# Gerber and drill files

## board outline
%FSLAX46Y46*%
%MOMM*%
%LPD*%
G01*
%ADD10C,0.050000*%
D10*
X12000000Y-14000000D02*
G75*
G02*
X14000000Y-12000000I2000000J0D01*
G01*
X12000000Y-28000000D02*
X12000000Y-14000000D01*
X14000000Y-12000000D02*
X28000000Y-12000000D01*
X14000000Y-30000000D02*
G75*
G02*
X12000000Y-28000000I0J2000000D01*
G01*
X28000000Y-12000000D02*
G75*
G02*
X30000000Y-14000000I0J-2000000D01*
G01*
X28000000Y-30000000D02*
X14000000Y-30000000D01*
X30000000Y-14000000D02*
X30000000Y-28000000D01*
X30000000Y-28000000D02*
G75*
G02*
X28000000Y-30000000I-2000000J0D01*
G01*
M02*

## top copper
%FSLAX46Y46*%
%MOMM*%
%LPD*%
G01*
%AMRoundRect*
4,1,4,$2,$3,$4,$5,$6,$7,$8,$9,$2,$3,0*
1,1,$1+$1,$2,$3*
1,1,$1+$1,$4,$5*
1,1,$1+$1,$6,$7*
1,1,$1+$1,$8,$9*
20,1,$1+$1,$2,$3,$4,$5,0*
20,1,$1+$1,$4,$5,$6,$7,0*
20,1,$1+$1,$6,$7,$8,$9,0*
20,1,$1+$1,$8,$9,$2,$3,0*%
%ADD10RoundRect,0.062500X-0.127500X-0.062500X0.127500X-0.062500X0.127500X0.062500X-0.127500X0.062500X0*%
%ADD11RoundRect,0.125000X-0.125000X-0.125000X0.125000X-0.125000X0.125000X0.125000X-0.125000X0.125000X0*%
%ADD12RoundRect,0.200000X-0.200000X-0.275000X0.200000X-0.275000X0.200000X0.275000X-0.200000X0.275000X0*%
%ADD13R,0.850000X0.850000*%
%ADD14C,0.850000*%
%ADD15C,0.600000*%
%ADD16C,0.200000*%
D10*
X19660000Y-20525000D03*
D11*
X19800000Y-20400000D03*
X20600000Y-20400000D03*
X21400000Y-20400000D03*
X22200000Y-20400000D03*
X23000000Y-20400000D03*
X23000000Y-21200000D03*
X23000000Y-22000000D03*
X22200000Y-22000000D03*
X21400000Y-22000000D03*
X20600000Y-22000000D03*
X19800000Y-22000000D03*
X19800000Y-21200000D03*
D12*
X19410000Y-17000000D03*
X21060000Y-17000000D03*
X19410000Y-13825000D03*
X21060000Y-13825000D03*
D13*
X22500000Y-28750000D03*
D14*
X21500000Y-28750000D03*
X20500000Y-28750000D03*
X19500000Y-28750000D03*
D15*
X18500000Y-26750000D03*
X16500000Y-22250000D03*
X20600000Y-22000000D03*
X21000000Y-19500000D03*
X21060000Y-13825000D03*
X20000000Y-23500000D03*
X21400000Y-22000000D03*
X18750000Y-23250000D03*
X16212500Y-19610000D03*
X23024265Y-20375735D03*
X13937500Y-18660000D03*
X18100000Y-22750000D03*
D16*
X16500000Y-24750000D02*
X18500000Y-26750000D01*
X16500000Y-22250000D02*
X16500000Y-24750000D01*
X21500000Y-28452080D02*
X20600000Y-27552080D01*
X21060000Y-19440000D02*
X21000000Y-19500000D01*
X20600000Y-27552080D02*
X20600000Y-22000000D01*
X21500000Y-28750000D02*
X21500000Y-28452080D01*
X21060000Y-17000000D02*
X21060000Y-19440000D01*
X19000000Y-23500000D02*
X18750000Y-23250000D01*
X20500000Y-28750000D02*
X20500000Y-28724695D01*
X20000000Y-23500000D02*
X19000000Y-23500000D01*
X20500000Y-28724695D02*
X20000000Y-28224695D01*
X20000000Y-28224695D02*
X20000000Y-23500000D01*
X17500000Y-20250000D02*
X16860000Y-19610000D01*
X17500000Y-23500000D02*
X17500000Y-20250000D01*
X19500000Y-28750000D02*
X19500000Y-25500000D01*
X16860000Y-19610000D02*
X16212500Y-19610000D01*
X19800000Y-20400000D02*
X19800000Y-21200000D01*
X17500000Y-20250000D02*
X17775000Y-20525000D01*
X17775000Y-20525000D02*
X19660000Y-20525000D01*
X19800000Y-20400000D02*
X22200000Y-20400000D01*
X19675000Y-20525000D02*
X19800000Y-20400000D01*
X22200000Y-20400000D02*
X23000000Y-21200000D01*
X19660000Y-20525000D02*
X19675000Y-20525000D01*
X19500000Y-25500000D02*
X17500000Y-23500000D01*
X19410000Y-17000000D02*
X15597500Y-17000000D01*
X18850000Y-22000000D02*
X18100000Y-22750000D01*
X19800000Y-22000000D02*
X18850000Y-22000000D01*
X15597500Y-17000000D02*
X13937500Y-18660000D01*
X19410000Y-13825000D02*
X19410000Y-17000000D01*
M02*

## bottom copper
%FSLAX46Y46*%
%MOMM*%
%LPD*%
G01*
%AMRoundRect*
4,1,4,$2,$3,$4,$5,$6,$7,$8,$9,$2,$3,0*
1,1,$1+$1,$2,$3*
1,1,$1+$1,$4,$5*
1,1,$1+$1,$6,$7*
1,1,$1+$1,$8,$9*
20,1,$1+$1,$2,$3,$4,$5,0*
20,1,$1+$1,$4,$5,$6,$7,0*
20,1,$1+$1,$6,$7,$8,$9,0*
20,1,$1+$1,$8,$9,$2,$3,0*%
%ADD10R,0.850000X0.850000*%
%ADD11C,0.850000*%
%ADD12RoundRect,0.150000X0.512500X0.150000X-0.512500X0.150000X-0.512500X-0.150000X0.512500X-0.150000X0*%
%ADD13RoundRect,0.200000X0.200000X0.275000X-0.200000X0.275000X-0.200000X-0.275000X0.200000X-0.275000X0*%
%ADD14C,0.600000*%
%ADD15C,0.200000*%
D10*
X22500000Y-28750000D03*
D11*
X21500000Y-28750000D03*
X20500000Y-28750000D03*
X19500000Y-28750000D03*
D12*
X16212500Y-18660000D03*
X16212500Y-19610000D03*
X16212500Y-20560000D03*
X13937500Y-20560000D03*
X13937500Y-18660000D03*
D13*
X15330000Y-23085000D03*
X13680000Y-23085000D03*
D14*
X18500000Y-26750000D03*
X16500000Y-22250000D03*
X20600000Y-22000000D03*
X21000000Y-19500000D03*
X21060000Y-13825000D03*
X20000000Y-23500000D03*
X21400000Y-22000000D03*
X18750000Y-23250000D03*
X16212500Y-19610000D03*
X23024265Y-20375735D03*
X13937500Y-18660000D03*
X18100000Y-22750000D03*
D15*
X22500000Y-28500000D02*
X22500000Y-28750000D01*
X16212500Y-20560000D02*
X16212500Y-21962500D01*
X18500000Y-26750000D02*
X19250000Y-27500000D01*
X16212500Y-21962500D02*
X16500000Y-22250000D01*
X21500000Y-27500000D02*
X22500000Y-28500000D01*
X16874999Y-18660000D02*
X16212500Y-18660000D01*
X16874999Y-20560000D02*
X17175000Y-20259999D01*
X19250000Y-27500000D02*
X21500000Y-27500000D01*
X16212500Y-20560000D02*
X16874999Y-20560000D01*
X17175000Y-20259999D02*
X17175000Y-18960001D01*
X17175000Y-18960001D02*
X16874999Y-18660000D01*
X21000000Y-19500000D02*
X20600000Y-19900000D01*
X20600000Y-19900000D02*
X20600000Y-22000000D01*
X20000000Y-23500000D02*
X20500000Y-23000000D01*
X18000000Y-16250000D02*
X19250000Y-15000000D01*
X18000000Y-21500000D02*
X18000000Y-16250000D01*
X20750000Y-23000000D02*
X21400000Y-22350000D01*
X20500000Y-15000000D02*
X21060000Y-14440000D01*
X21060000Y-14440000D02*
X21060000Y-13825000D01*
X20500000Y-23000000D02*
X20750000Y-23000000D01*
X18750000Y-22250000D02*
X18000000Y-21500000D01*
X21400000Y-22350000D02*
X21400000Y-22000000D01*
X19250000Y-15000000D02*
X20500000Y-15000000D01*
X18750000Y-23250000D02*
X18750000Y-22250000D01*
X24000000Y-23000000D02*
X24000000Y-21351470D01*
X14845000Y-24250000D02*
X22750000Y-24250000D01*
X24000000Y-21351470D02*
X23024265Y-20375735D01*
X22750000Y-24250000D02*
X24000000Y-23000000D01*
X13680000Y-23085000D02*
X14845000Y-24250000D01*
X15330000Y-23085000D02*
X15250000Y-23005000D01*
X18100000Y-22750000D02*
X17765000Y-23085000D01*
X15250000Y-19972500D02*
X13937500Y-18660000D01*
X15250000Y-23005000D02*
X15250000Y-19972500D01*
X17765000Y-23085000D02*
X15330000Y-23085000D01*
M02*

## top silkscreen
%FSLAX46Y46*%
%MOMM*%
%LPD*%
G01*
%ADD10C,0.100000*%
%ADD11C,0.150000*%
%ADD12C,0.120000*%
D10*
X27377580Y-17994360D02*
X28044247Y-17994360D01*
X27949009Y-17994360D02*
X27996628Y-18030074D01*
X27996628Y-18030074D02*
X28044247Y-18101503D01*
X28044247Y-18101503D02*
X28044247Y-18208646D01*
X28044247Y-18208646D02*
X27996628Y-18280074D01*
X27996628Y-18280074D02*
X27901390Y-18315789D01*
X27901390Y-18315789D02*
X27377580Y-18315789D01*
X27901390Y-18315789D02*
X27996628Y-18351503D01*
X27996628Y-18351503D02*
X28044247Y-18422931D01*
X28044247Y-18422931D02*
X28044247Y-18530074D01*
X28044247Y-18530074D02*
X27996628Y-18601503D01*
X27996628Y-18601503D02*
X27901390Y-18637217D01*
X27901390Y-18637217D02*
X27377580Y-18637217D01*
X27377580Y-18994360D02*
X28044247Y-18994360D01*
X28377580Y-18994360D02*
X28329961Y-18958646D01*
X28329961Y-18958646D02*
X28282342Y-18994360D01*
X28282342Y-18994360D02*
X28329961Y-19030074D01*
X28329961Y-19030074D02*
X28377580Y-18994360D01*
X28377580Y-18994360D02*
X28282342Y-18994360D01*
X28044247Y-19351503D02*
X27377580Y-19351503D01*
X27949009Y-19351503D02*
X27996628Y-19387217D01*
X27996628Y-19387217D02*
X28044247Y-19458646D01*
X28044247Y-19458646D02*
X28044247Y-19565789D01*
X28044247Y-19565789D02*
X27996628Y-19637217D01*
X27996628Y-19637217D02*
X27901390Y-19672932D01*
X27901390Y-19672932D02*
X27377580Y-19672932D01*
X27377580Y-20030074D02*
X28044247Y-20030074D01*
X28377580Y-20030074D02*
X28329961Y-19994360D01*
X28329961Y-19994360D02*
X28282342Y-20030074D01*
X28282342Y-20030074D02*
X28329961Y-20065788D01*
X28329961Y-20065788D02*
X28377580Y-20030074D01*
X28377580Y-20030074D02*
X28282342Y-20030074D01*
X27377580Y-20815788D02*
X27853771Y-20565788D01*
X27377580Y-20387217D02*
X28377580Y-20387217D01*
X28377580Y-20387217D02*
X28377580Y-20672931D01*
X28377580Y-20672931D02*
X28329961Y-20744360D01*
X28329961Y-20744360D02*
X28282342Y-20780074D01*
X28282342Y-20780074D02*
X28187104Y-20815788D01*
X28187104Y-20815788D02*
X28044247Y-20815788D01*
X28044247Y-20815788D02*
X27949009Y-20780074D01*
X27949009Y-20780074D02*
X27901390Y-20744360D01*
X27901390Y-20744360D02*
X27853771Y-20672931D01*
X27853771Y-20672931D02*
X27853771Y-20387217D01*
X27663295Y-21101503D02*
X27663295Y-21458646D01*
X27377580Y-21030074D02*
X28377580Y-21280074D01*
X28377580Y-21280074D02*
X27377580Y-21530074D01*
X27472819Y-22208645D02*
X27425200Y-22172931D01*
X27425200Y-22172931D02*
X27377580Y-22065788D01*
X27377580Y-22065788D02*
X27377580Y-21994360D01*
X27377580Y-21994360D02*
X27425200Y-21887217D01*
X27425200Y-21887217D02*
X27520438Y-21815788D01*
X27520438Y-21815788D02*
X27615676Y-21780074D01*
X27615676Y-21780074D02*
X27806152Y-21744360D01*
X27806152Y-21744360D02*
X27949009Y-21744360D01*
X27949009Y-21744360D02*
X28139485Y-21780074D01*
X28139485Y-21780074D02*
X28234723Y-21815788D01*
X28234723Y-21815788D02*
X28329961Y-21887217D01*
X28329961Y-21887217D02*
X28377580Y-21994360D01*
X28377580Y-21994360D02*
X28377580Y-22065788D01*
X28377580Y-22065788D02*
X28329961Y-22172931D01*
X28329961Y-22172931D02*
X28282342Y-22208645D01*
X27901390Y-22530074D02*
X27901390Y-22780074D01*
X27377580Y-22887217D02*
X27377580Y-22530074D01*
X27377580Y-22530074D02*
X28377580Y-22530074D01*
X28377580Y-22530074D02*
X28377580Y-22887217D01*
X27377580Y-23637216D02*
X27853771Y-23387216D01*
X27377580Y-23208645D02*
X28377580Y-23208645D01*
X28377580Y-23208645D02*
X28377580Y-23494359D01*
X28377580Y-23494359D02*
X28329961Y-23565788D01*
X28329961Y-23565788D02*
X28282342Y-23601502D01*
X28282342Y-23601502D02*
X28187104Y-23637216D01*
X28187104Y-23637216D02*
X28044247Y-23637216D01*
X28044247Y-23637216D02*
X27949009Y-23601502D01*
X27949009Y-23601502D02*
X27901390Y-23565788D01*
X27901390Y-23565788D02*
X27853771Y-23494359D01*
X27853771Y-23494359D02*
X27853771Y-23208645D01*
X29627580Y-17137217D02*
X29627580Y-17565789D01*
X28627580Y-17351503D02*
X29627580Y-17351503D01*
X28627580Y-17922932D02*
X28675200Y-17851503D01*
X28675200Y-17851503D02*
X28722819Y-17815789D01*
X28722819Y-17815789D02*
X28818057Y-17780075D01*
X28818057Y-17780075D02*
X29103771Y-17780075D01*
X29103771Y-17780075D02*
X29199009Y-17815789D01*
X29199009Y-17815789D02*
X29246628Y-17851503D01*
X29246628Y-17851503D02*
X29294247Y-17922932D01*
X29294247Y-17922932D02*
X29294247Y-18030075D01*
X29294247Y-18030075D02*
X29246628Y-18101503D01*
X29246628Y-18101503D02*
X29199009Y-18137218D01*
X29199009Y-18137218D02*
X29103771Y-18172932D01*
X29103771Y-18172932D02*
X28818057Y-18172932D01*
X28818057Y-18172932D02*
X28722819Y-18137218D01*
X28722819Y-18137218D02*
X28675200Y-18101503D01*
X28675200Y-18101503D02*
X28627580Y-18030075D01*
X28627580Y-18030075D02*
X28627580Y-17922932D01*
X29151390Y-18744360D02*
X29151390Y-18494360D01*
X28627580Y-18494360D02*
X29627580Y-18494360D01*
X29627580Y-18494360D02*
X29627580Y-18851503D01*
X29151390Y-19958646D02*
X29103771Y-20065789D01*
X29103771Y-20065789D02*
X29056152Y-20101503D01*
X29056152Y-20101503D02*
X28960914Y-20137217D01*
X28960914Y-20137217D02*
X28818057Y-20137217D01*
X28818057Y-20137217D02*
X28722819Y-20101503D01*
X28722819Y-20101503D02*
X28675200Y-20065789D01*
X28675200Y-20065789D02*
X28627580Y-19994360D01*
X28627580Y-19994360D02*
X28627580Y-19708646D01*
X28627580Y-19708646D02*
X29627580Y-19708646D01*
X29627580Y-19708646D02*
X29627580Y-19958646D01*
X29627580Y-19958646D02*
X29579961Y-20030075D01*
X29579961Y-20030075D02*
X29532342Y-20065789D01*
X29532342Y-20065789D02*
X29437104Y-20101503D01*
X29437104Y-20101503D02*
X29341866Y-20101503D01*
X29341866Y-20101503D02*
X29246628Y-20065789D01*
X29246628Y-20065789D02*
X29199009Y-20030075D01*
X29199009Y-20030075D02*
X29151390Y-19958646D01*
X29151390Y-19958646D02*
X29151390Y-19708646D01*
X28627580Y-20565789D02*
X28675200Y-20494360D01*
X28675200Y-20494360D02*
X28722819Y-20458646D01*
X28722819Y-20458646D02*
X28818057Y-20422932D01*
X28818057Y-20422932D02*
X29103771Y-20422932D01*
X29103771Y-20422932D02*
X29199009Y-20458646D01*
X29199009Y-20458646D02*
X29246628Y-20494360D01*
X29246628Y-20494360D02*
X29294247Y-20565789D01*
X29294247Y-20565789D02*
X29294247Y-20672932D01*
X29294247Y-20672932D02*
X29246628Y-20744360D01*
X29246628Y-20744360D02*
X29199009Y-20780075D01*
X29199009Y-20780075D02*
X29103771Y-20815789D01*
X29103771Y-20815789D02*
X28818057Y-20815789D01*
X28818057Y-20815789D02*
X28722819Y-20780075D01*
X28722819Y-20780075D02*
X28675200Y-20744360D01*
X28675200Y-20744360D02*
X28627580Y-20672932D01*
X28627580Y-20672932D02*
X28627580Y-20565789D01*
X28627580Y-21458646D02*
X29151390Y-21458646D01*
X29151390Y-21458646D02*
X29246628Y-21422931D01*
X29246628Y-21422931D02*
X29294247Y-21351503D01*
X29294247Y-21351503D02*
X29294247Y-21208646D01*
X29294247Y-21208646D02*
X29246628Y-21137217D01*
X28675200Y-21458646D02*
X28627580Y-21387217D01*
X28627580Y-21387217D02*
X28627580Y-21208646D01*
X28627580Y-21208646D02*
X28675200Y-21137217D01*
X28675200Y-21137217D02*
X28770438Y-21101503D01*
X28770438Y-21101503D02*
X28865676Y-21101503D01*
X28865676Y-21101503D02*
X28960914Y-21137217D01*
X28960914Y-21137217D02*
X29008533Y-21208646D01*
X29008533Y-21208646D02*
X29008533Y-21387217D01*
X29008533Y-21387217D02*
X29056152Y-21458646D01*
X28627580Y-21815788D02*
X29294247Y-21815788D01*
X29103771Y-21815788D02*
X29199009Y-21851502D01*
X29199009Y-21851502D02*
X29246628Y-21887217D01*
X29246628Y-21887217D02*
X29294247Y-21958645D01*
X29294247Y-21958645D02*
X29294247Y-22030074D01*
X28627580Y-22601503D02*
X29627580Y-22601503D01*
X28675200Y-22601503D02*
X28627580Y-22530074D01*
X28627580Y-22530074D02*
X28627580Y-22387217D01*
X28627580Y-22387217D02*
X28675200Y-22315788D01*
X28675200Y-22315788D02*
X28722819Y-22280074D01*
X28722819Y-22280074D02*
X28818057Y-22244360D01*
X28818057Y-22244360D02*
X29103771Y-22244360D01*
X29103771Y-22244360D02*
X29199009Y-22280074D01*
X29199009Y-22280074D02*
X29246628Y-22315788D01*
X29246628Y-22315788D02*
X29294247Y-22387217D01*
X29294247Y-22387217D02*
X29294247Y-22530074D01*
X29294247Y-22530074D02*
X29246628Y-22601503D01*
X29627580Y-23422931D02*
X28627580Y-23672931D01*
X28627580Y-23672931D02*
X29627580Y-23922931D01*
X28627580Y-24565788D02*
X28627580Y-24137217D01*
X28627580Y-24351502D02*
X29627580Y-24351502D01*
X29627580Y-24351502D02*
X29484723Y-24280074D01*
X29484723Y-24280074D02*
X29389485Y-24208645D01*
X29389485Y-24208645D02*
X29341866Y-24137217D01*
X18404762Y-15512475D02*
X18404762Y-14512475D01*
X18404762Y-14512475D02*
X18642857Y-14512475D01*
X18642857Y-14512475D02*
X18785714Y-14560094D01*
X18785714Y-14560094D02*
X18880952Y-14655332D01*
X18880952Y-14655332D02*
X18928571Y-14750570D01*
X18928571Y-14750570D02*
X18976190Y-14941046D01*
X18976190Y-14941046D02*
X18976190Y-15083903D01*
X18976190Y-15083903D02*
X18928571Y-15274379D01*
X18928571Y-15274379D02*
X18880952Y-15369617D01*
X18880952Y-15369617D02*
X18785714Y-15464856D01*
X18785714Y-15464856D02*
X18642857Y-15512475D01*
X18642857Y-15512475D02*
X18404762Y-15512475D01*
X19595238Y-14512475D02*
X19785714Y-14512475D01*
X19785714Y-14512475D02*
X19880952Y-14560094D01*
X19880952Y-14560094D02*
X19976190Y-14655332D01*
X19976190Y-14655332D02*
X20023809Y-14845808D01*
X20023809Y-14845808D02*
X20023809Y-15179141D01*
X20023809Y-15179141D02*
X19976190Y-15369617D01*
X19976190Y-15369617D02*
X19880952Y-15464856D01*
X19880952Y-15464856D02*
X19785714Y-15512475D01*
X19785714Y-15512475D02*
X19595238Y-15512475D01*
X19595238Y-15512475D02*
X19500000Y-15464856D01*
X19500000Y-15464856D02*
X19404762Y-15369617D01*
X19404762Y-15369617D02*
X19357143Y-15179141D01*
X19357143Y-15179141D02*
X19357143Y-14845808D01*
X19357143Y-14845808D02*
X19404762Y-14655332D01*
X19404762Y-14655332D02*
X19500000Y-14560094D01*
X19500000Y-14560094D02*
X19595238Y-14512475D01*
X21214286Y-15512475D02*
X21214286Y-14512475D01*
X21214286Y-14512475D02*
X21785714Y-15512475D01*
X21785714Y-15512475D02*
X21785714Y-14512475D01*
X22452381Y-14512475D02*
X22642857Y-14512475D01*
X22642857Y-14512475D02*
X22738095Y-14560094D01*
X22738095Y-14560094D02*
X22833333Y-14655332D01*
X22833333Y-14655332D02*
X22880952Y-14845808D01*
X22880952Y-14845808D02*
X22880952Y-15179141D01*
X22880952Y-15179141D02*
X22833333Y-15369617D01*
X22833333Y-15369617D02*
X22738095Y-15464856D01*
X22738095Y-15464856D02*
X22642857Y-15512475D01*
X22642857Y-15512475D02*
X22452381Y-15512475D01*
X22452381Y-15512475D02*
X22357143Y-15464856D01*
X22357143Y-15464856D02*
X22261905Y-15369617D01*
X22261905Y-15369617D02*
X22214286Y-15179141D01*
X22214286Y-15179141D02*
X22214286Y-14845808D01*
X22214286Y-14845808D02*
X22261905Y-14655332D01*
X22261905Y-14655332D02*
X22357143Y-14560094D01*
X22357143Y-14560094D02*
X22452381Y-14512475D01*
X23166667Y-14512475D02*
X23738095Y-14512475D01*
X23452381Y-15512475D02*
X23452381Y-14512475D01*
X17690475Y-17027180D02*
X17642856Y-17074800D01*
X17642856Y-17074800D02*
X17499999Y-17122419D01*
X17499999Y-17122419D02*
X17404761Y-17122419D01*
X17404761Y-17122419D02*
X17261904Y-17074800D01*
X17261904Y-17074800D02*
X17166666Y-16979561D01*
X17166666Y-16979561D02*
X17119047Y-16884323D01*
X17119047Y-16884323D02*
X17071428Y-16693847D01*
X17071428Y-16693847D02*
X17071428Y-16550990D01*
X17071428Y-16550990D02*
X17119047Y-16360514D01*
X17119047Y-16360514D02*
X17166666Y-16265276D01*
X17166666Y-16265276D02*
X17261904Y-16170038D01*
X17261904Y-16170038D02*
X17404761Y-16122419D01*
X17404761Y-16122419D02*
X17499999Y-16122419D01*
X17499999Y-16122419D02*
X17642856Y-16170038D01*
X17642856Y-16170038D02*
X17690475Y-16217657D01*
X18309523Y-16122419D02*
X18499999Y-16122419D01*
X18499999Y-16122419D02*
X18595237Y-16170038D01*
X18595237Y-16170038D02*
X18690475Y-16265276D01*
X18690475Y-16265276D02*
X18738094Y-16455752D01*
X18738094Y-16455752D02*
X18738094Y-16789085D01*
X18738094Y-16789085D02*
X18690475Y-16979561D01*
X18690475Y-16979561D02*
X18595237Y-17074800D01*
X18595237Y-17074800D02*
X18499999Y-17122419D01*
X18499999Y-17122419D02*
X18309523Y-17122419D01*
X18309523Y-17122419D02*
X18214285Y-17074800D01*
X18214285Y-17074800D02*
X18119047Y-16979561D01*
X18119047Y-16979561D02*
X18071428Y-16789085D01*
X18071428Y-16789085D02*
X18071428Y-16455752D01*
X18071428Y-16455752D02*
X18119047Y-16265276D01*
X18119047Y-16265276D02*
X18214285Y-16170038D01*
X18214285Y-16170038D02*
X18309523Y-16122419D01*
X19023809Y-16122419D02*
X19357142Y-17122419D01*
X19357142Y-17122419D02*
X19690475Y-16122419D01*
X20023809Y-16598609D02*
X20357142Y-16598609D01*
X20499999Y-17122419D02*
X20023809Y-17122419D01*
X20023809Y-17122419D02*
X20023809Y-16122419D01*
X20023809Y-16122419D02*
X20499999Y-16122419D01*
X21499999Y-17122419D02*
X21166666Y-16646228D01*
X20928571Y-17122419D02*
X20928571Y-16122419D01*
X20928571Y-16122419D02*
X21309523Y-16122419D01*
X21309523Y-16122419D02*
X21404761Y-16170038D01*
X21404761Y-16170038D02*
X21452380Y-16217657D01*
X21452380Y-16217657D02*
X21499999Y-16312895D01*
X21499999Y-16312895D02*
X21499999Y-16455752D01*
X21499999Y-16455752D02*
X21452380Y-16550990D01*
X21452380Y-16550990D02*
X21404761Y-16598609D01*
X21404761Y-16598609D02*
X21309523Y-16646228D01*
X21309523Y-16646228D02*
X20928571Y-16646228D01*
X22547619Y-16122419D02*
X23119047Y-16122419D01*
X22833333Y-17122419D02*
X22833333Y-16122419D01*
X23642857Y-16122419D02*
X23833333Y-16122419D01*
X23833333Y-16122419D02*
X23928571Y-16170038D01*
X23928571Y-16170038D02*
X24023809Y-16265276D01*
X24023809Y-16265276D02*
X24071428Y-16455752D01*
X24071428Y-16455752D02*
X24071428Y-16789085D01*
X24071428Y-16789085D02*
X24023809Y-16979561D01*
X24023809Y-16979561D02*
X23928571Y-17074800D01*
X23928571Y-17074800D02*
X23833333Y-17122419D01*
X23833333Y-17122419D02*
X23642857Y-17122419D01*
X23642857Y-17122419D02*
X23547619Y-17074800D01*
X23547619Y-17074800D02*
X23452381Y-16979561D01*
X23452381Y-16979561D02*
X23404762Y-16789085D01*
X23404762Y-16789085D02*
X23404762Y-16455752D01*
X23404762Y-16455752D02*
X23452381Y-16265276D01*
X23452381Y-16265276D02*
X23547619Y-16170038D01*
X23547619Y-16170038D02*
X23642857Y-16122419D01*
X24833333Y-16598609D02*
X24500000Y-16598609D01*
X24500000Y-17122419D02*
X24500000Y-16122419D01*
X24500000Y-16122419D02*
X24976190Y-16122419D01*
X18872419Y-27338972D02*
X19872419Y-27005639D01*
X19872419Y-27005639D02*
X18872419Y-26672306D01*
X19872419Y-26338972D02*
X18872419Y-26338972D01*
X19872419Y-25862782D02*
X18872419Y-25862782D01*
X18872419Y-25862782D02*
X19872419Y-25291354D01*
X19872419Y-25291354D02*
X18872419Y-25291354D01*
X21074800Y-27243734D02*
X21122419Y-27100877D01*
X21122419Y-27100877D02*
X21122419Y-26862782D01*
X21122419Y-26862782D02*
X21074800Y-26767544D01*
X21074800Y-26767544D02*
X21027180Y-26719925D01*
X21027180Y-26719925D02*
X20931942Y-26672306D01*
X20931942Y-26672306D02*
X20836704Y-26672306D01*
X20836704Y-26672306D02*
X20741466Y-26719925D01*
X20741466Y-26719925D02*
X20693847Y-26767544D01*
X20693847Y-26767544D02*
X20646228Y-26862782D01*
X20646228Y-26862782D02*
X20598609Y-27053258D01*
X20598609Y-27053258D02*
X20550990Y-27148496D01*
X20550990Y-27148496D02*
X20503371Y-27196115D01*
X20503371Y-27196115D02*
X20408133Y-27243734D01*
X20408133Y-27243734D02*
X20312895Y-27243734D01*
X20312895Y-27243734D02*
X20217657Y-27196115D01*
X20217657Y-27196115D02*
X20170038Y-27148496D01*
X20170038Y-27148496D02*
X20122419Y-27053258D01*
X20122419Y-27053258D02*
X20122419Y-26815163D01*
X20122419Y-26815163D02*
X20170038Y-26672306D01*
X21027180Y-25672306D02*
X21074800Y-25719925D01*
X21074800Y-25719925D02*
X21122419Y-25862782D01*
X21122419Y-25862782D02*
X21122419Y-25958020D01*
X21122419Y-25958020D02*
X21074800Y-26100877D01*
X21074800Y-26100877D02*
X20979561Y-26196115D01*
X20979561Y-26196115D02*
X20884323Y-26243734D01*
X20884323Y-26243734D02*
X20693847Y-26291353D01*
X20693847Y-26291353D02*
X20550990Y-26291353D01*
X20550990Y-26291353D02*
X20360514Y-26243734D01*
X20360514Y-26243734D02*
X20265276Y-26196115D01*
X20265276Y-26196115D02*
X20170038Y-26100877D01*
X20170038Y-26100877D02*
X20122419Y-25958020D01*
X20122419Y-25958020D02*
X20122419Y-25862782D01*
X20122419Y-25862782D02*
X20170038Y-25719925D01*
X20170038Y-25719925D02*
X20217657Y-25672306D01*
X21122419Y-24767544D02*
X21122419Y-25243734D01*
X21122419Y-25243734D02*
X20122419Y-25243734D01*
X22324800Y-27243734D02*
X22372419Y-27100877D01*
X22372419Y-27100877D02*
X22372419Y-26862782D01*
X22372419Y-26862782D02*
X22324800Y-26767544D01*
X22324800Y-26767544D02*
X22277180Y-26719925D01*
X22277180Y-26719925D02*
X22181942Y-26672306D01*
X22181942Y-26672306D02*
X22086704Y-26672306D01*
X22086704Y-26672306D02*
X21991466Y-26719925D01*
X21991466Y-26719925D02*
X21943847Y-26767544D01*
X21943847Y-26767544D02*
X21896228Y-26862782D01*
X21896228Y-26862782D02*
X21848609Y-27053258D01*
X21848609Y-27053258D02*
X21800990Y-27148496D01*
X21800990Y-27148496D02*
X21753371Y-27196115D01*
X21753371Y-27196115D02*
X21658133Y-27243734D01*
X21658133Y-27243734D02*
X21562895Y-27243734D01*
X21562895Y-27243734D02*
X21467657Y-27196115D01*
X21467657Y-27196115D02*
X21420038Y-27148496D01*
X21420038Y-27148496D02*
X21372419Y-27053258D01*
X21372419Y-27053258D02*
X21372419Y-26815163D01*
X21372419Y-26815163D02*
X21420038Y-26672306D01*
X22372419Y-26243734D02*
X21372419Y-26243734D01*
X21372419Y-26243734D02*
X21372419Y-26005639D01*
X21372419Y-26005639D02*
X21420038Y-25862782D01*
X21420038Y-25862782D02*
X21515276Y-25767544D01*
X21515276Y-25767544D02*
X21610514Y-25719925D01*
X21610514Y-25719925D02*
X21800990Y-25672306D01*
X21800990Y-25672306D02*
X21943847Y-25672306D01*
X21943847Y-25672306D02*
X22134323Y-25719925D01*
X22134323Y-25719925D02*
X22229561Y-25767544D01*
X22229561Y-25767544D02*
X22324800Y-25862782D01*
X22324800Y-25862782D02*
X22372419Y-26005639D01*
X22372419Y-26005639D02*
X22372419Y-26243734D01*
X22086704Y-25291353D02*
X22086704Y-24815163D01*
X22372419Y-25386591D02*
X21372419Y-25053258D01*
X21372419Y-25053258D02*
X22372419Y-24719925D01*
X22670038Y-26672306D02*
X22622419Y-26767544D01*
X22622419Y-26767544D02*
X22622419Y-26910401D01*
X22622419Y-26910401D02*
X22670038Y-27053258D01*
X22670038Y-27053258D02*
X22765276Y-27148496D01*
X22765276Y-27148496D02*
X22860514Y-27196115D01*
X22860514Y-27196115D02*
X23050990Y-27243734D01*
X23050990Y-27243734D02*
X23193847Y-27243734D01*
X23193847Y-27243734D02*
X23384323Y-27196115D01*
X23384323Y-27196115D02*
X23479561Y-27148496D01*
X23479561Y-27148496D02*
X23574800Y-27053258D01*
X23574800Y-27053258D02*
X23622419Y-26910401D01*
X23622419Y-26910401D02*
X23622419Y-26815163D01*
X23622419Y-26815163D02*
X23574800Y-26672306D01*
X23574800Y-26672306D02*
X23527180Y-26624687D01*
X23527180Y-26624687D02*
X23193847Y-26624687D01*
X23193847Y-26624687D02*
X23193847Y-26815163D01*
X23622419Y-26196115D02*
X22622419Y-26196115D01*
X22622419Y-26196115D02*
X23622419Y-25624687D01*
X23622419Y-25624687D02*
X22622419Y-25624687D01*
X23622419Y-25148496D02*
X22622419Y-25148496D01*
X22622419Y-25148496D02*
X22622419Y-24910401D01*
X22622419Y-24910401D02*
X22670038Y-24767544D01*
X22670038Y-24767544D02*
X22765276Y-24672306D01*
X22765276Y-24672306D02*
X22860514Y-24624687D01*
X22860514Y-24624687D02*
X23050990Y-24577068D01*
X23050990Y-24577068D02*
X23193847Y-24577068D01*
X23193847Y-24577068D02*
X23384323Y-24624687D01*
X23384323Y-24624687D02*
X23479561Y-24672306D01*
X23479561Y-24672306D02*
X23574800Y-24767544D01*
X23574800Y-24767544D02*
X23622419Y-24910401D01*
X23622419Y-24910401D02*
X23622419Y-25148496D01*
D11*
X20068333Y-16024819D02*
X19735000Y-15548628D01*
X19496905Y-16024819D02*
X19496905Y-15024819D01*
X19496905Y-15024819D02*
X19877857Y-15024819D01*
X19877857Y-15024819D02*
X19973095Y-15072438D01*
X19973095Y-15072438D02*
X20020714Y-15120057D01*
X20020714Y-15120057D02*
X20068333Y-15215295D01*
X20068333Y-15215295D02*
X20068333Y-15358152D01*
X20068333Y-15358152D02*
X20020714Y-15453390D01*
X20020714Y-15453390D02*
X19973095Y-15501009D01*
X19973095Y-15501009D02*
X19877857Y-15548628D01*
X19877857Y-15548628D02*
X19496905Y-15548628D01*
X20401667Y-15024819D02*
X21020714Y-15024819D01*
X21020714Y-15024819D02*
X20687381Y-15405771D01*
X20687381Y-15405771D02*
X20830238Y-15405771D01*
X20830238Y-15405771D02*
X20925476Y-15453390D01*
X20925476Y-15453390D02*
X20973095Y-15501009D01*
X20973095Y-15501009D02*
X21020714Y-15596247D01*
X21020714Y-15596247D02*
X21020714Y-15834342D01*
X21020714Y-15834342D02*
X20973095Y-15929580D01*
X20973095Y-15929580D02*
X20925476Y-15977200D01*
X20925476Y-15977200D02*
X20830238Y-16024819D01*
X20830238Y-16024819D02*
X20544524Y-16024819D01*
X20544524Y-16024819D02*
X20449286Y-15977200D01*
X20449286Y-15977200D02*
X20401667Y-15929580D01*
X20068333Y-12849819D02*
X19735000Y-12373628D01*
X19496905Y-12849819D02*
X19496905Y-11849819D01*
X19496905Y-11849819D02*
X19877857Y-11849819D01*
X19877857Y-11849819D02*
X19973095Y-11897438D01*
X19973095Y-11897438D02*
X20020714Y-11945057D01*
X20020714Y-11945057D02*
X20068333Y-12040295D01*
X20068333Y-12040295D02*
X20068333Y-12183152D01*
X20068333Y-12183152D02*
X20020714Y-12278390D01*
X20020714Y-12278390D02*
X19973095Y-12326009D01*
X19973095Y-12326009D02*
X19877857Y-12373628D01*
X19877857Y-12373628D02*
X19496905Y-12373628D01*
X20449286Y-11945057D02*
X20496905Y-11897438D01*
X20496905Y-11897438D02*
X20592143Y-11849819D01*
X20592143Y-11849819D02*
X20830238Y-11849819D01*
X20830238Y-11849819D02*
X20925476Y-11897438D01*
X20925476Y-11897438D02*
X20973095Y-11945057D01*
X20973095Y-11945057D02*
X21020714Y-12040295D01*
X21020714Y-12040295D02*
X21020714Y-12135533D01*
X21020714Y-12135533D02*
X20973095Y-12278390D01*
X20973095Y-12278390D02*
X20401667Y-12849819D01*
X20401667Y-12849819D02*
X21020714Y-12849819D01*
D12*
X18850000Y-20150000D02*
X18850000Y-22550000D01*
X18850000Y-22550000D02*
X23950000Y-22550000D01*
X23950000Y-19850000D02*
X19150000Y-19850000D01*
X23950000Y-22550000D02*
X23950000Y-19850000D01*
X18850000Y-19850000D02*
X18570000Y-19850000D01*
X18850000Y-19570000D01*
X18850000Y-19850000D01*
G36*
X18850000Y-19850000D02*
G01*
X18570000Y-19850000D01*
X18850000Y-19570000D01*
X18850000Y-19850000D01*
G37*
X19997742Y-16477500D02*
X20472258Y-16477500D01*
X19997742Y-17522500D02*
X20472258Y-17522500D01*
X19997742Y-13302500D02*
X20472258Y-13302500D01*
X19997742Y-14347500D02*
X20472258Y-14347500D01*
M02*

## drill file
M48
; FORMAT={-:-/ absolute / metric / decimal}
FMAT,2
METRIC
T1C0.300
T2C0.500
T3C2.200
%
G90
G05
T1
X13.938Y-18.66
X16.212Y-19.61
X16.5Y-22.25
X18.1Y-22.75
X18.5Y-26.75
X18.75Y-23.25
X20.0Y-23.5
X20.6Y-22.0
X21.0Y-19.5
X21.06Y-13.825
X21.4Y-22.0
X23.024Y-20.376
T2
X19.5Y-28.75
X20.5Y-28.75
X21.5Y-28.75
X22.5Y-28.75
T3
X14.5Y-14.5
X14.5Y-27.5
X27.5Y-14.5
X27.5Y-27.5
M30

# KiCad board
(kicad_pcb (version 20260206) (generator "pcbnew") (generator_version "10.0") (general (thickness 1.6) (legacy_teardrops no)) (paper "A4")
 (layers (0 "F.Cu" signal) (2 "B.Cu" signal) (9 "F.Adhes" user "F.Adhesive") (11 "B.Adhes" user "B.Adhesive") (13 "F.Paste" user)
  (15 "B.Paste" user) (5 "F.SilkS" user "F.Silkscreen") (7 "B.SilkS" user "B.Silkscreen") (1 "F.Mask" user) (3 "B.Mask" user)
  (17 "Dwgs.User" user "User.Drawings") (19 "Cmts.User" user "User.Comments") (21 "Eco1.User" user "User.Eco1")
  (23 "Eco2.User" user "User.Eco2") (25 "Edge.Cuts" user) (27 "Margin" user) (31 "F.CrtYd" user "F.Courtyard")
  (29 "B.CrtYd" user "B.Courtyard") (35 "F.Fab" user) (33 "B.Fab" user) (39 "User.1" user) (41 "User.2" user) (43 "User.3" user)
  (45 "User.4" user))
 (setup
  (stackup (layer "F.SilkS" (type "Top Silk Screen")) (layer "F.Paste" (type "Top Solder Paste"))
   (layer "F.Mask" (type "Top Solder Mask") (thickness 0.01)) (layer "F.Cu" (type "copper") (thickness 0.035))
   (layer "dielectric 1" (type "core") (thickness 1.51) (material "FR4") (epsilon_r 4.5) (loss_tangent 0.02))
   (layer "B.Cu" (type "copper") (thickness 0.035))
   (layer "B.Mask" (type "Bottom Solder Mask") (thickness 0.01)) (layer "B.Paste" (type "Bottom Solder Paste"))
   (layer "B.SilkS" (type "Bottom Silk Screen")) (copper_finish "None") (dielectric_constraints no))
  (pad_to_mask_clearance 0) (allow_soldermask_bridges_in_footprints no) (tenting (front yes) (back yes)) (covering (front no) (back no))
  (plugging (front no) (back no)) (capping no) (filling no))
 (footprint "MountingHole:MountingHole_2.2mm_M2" (layer "F.Cu") (at 27.5 14.5)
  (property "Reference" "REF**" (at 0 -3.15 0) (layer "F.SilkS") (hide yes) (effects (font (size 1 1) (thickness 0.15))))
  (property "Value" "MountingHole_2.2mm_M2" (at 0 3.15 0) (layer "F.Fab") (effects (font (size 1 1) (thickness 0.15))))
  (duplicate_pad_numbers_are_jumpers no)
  (pad "" np_thru_hole circle (at 0 0) (size 2.2 2.2) (drill 2.2) (layers "*.Cu" "*.Mask")))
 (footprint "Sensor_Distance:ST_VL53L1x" (layer "F.Cu") (at 21.4 21.2)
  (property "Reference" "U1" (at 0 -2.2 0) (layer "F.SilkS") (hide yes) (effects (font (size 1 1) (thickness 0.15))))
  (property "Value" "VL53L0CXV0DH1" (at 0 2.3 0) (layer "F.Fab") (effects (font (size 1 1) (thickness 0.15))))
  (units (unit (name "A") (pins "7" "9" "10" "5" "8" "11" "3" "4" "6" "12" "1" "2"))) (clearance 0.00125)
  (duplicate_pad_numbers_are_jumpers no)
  (fp_line (start -2.55 -1.05) (end -2.55 1.35) (stroke (width 0.12) (type solid)) (layer "F.SilkS"))
  (fp_line (start -2.55 1.35) (end 2.55 1.35) (stroke (width 0.12) (type solid)) (layer "F.SilkS"))
  (fp_line (start 2.55 -1.35) (end -2.25 -1.35) (stroke (width 0.12) (type solid)) (layer "F.SilkS"))
  (fp_line (start 2.55 1.35) (end 2.55 -1.35) (stroke (width 0.12) (type solid)) (layer "F.SilkS"))
  (fp_poly
   (pts (xy -2.55 -1.35) (xy -2.83 -1.35) (xy -2.55 -1.63) (xy -2.55 -1.35)) (stroke (width 0.12) (type solid)) (fill yes) (layer "F.SilkS"))
  (pad "1" smd roundrect (at -1.74 -0.675) (size 0.38 0.25) (layers "F.Cu" "F.Mask" "F.Paste") (roundrect_rratio 0.25)
   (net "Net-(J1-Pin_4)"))
  (pad "1" smd roundrect (at -1.6 -0.8) (size 0.5 0.5) (layers "F.Cu" "F.Mask" "F.Paste") (roundrect_rratio 0.25) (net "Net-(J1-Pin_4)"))
  (pad "2" smd roundrect (at -0.8 -0.8) (size 0.5 0.5) (layers "F.Cu" "F.Mask" "F.Paste") (roundrect_rratio 0.25) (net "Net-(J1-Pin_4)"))
  (pad "3" smd roundrect (at 0 -0.8) (size 0.5 0.5) (layers "F.Cu" "F.Mask" "F.Paste") (roundrect_rratio 0.25) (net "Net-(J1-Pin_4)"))
  (pad "4" smd roundrect (at 0.8 -0.8) (size 0.5 0.5) (layers "F.Cu" "F.Mask" "F.Paste") (roundrect_rratio 0.25) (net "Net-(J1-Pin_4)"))
  (pad "5" smd roundrect (at 1.6 -0.8) (size 0.5 0.5) (layers "F.Cu" "F.Mask" "F.Paste") (roundrect_rratio 0.25) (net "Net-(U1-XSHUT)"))
  (pad "6" smd roundrect (at 1.6 0) (size 0.5 0.5) (layers "F.Cu" "F.Mask" "F.Paste") (roundrect_rratio 0.25) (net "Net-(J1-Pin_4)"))
  (pad "7" smd roundrect (at 1.6 0.8) (size 0.5 0.5) (layers "F.Cu" "F.Mask" "F.Paste") (roundrect_rratio 0.25)
   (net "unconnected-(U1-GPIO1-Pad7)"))
  (pad "8" smd roundrect (at 0.8 0.8) (size 0.5 0.5) (layers "F.Cu" "F.Mask" "F.Paste") (roundrect_rratio 0.25)
   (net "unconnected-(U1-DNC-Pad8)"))
  (pad "9" smd roundrect (at 0 0.8) (size 0.5 0.5) (layers "F.Cu" "F.Mask" "F.Paste") (roundrect_rratio 0.25) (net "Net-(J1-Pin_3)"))
  (pad "10" smd roundrect (at -0.8 0.8) (size 0.5 0.5) (layers "F.Cu" "F.Mask" "F.Paste") (roundrect_rratio 0.25) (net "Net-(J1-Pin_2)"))
  (pad "11" smd roundrect (at -1.6 0.8) (size 0.5 0.5) (layers "F.Cu" "F.Mask" "F.Paste") (roundrect_rratio 0.25) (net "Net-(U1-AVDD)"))
  (pad "12" smd roundrect (at -1.6 0) (size 0.5 0.5) (layers "F.Cu" "F.Mask" "F.Paste") (roundrect_rratio 0.25) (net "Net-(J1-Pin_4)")))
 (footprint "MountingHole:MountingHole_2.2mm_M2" (layer "F.Cu") (at 27.5 27.5)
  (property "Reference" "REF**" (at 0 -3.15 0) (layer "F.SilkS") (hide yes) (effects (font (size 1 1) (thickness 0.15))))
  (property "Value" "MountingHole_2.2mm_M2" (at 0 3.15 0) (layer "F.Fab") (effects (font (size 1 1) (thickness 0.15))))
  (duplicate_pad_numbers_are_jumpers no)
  (pad "" np_thru_hole circle (at 0 0) (size 2.2 2.2) (drill 2.2) (layers "*.Cu" "*.Mask")))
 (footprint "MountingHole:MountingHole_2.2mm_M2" (layer "F.Cu") (at 14.5 14.5)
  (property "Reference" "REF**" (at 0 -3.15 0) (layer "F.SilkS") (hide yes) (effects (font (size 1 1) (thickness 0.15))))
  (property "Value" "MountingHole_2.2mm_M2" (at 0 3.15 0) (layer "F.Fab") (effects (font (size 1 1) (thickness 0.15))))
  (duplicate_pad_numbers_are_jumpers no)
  (pad "" np_thru_hole circle (at 0 0) (size 2.2 2.2) (drill 2.2) (layers "*.Cu" "*.Mask")))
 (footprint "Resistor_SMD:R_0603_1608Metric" (layer "F.Cu") (at 20.235 17)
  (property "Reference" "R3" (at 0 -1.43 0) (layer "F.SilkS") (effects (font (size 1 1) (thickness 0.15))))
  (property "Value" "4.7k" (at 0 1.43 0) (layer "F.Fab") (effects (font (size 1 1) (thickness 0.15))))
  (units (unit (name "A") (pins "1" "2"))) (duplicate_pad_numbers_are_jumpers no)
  (fp_line (start -0.237258 -0.5225) (end 0.237258 -0.5225) (stroke (width 0.12) (type solid)) (layer "F.SilkS"))
  (fp_line (start -0.237258 0.5225) (end 0.237258 0.5225) (stroke (width 0.12) (type solid)) (layer "F.SilkS"))
  (pad "1" smd roundrect (at -0.825 0) (size 0.8 0.95) (layers "F.Cu" "F.Mask" "F.Paste") (roundrect_rratio 0.25) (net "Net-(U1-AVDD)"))
  (pad "2" smd roundrect (at 0.825 0) (size 0.8 0.95) (layers "F.Cu" "F.Mask" "F.Paste") (roundrect_rratio 0.25) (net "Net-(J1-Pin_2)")))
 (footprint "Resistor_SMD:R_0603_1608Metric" (layer "F.Cu") (at 20.235 13.825)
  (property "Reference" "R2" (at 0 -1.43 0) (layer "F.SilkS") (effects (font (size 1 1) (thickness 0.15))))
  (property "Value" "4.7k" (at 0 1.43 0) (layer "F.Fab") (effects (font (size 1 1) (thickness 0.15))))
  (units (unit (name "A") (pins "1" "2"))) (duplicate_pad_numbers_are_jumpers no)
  (fp_line (start -0.237258 -0.5225) (end 0.237258 -0.5225) (stroke (width 0.12) (type solid)) (layer "F.SilkS"))
  (fp_line (start -0.237258 0.5225) (end 0.237258 0.5225) (stroke (width 0.12) (type solid)) (layer "F.SilkS"))
  (pad "1" smd roundrect (at -0.825 0) (size 0.8 0.95) (layers "F.Cu" "F.Mask" "F.Paste") (roundrect_rratio 0.25) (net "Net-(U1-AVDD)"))
  (pad "2" smd roundrect (at 0.825 0) (size 0.8 0.95) (layers "F.Cu" "F.Mask" "F.Paste") (roundrect_rratio 0.25) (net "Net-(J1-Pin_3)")))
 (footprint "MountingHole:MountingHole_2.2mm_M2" (layer "F.Cu") (at 14.5 27.5)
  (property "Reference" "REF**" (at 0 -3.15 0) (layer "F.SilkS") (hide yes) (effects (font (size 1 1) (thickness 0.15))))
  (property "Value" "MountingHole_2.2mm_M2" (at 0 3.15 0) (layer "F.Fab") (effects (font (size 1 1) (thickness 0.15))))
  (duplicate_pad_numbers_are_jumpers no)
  (pad "" np_thru_hole circle (at 0 0) (size 2.2 2.2) (drill 2.2) (layers "*.Cu" "*.Mask")))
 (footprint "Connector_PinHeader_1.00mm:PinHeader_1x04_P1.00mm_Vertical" (layer "B.Cu") (at 22.5 28.75 90)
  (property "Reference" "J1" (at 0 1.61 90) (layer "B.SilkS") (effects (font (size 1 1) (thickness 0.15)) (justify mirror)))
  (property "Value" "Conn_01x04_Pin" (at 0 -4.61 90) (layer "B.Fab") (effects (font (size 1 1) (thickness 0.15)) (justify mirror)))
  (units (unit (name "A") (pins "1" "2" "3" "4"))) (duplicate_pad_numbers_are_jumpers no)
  (pad "1" thru_hole rect (at 0 0 90) (size 0.85 0.85) (drill 0.5) (layers "*.Cu" "*.Mask") (remove_unused_layers no) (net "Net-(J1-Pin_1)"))
  (pad "2" thru_hole circle (at 0 -1 90) (size 0.85 0.85) (drill 0.5) (layers "*.Cu" "*.Mask") (remove_unused_layers no)
   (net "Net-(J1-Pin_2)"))
  (pad "3" thru_hole circle (at 0 -2 90) (size 0.85 0.85) (drill 0.5) (layers "*.Cu" "*.Mask") (remove_unused_layers no)
   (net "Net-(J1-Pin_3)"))
  (pad "4" thru_hole circle (at 0 -3 90) (size 0.85 0.85) (drill 0.5) (layers "*.Cu" "*.Mask") (remove_unused_layers no)
   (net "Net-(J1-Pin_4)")))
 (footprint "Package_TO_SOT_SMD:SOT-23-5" (layer "B.Cu") (at 15.075 19.61 180)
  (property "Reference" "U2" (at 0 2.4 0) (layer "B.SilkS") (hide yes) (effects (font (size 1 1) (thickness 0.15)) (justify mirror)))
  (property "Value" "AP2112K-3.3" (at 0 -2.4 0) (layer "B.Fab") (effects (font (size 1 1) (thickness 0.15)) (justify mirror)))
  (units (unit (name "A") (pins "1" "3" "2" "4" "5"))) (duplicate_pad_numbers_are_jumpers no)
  (pad "1" smd roundrect (at -1.1375 0.95 180) (size 1.325 0.6) (layers "B.Cu" "B.Mask" "B.Paste") (roundrect_rratio 0.25)
   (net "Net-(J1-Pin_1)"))
  (pad "2" smd roundrect (at -1.1375 0 180) (size 1.325 0.6) (layers "B.Cu" "B.Mask" "B.Paste") (roundrect_rratio 0.25)
   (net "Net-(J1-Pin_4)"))
  (pad "3" smd roundrect (at -1.1375 -0.95 180) (size 1.325 0.6) (layers "B.Cu" "B.Mask" "B.Paste") (roundrect_rratio 0.25)
   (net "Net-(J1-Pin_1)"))
  (pad "4" smd roundrect (at 1.1375 -0.95 180) (size 1.325 0.6) (layers "B.Cu" "B.Mask" "B.Paste") (roundrect_rratio 0.25)
   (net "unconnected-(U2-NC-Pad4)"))
  (pad "5" smd roundrect (at 1.1375 0.95 180) (size 1.325 0.6) (layers "B.Cu" "B.Mask" "B.Paste") (roundrect_rratio 0.25)
   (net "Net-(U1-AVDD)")))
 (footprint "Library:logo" (layer "B.Cu") (at 21 21.5 180)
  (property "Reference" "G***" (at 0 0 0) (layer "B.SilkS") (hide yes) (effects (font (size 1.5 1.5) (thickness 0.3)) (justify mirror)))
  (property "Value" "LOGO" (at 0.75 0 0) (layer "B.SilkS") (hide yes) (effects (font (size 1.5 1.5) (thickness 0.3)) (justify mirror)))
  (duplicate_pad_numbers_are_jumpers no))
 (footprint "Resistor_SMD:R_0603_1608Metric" (layer "B.Cu") (at 14.505 23.085 180)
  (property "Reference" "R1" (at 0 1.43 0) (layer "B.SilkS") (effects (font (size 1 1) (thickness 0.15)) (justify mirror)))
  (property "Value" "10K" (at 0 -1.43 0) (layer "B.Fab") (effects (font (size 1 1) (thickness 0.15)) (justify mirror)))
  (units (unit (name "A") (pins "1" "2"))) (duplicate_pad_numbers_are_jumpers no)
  (pad "1" smd roundrect (at -0.825 0 180) (size 0.8 0.95) (layers "B.Cu" "B.Mask" "B.Paste") (roundrect_rratio 0.25) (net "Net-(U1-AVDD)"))
  (pad "2" smd roundrect (at 0.825 0 180) (size 0.8 0.95) (layers "B.Cu" "B.Mask" "B.Paste") (roundrect_rratio 0.25) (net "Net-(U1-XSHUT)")))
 (gr_arc (start 12 14) (mid 12.585786 12.585786) (end 14 12) (stroke (width 0.05) (type default)) (layer "Edge.Cuts"))
 (gr_line (start 12 28) (end 12 14) (stroke (width 0.05) (type default)) (layer "Edge.Cuts"))
 (gr_line (start 14 12) (end 28 12) (stroke (width 0.05) (type default)) (layer "Edge.Cuts"))
 (gr_arc (start 14 30) (mid 12.585786 29.414214) (end 12 28) (stroke (width 0.05) (type default)) (layer "Edge.Cuts"))
 (gr_arc (start 28 12) (mid 29.414214 12.585786) (end 30 14) (stroke (width 0.05) (type default)) (layer "Edge.Cuts"))
 (gr_line (start 28 30) (end 14 30) (stroke (width 0.05) (type default)) (layer "Edge.Cuts"))
 (gr_line (start 30 14) (end 30 28) (stroke (width 0.05) (type default)) (layer "Edge.Cuts"))
 (gr_arc (start 30 28) (mid 29.414214 29.414214) (end 28 30) (stroke (width 0.05) (type default)) (layer "Edge.Cuts"))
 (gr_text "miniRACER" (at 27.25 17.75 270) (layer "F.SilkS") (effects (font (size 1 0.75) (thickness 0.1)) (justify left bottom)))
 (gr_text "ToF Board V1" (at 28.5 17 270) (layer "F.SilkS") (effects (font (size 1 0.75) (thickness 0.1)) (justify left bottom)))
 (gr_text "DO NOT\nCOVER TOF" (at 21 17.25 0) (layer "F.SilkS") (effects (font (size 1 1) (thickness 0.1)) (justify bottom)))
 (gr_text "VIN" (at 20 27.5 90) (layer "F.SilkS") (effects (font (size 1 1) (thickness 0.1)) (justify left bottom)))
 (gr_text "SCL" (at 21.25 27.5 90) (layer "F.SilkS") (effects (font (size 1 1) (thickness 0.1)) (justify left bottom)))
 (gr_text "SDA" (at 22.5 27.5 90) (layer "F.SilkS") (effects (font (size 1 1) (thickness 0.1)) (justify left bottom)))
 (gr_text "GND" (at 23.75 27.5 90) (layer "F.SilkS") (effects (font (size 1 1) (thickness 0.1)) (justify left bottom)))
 (segment (start 16.5 24.75) (end 18.5 26.75) (width 0.2) (layer "F.Cu") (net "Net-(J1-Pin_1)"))
 (segment (start 16.5 22.25) (end 16.5 24.75) (width 0.2) (layer "F.Cu") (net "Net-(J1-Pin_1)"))
 (via (at 18.5 26.75) (size 0.6) (drill 0.3) (layers "F.Cu" "B.Cu") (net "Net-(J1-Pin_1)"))
 (via (at 16.5 22.25) (size 0.6) (drill 0.3) (layers "F.Cu" "B.Cu") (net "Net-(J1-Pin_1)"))
 (segment (start 22.5 28.5) (end 22.5 28.75) (width 0.2) (layer "B.Cu") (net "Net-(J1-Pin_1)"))
 (segment (start 16.2125 20.56) (end 16.2125 21.9625) (width 0.2) (layer "B.Cu") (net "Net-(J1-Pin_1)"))
 (segment (start 18.5 26.75) (end 19.25 27.5) (width 0.2) (layer "B.Cu") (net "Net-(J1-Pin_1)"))
 (segment (start 16.2125 21.9625) (end 16.5 22.25) (width 0.2) (layer "B.Cu") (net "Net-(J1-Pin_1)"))
 (segment (start 21.5 27.5) (end 22.5 28.5) (width 0.2) (layer "B.Cu") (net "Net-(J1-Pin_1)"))
 (segment (start 16.874999 18.66) (end 16.2125 18.66) (width 0.2) (layer "B.Cu") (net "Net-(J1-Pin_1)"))
 (segment (start 16.874999 20.56) (end 17.175 20.259999) (width 0.2) (layer "B.Cu") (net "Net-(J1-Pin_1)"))
 (segment (start 19.25 27.5) (end 21.5 27.5) (width 0.2) (layer "B.Cu") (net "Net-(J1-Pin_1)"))
 (segment (start 16.2125 20.56) (end 16.874999 20.56) (width 0.2) (layer "B.Cu") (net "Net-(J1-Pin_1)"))
 (segment (start 17.175 20.259999) (end 17.175 18.960001) (width 0.2) (layer "B.Cu") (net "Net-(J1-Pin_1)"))
 (segment (start 17.175 18.960001) (end 16.874999 18.66) (width 0.2) (layer "B.Cu") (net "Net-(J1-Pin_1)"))
 (segment (start 21.5 28.45208) (end 20.6 27.55208) (width 0.2) (layer "F.Cu") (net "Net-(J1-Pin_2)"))
 (segment (start 21.06 19.44) (end 21 19.5) (width 0.2) (layer "F.Cu") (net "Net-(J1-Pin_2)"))
 (segment (start 20.6 27.55208) (end 20.6 22) (width 0.2) (layer "F.Cu") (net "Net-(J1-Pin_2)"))
 (segment (start 21.5 28.75) (end 21.5 28.45208) (width 0.2) (layer "F.Cu") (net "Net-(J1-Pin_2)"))
 (segment (start 21.06 17) (end 21.06 19.44) (width 0.2) (layer "F.Cu") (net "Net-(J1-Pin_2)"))
 (via (at 20.6 22) (size 0.6) (drill 0.3) (layers "F.Cu" "B.Cu") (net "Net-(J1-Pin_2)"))
 (via (at 21 19.5) (size 0.6) (drill 0.3) (layers "F.Cu" "B.Cu") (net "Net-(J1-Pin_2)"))
 (segment (start 21 19.5) (end 20.6 19.9) (width 0.2) (layer "B.Cu") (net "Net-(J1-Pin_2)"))
 (segment (start 20.6 19.9) (end 20.6 22) (width 0.2) (layer "B.Cu") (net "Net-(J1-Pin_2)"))
 (segment (start 19 23.5) (end 18.75 23.25) (width 0.2) (layer "F.Cu") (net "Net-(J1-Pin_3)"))
 (segment (start 20.5 28.75) (end 20.5 28.724695) (width 0.2) (layer "F.Cu") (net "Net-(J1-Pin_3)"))
 (segment (start 20 23.5) (end 19 23.5) (width 0.2) (layer "F.Cu") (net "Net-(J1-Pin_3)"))
 (segment (start 20.5 28.724695) (end 20 28.224695) (width 0.2) (layer "F.Cu") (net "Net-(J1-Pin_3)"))
 (segment (start 20 28.224695) (end 20 23.5) (width 0.2) (layer "F.Cu") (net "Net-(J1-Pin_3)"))
 (via (at 21.06 13.825) (size 0.6) (drill 0.3) (layers "F.Cu" "B.Cu") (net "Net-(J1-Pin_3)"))
 (via (at 20 23.5) (size 0.6) (drill 0.3) (layers "F.Cu" "B.Cu") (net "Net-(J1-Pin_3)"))
 (via (at 21.4 22) (size 0.6) (drill 0.3) (layers "F.Cu" "B.Cu") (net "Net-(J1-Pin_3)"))
 (via (at 18.75 23.25) (size 0.6) (drill 0.3) (layers "F.Cu" "B.Cu") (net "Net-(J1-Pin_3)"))
 (segment (start 20 23.5) (end 20.5 23) (width 0.2) (layer "B.Cu") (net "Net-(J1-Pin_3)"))
 (segment (start 18 16.25) (end 19.25 15) (width 0.2) (layer "B.Cu") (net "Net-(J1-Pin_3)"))
 (segment (start 18 21.5) (end 18 16.25) (width 0.2) (layer "B.Cu") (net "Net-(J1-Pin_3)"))
 (segment (start 20.75 23) (end 21.4 22.35) (width 0.2) (layer "B.Cu") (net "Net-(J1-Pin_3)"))
 (segment (start 20.5 15) (end 21.06 14.44) (width 0.2) (layer "B.Cu") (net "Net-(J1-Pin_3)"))
 (segment (start 21.06 14.44) (end 21.06 13.825) (width 0.2) (layer "B.Cu") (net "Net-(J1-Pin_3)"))
 (segment (start 20.5 23) (end 20.75 23) (width 0.2) (layer "B.Cu") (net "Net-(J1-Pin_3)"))
 (segment (start 18.75 22.25) (end 18 21.5) (width 0.2) (layer "B.Cu") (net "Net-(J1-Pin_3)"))
 (segment (start 21.4 22.35) (end 21.4 22) (width 0.2) (layer "B.Cu") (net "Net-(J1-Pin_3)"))
 (segment (start 19.25 15) (end 20.5 15) (width 0.2) (layer "B.Cu") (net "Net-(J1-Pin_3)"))
 (segment (start 18.75 23.25) (end 18.75 22.25) (width 0.2) (layer "B.Cu") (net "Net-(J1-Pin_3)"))
 (segment (start 17.5 20.25) (end 16.86 19.61) (width 0.2) (layer "F.Cu") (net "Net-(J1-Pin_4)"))
 (segment (start 17.5 23.5) (end 17.5 20.25) (width 0.2) (layer "F.Cu") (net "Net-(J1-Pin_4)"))
 (segment (start 19.5 28.75) (end 19.5 25.5) (width 0.2) (layer "F.Cu") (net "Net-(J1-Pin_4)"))
 (segment (start 16.86 19.61) (end 16.2125 19.61) (width 0.2) (layer "F.Cu") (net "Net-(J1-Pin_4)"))
 (segment (start 19.8 20.4) (end 19.8 21.2) (width 0.2) (layer "F.Cu") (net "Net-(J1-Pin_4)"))
 (segment (start 17.5 20.25) (end 17.775 20.525) (width 0.2) (layer "F.Cu") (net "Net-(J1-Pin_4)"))
 (segment (start 17.775 20.525) (end 19.66 20.525) (width 0.2) (layer "F.Cu") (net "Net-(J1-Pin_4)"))
 (segment (start 19.8 20.4) (end 22.2 20.4) (width 0.2) (layer "F.Cu") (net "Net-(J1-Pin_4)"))
 (segment (start 19.675 20.525) (end 19.8 20.4) (width 0.2) (layer "F.Cu") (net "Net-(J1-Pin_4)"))
 (segment (start 22.2 20.4) (end 23 21.2) (width 0.2) (layer "F.Cu") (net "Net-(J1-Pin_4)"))
 (segment (start 19.66 20.525) (end 19.675 20.525) (width 0.2) (layer "F.Cu") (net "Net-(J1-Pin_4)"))
 (segment (start 19.5 25.5) (end 17.5 23.5) (width 0.2) (layer "F.Cu") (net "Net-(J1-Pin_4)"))
 (via (at 16.2125 19.61) (size 0.6) (drill 0.3) (layers "F.Cu" "B.Cu") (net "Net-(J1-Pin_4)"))
 (via (at 23.024265 20.375735) (size 0.6) (drill 0.3) (layers "F.Cu" "B.Cu") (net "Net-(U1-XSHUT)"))
 (segment (start 24 23) (end 24 21.35147) (width 0.2) (layer "B.Cu") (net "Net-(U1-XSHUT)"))
 (segment (start 14.845 24.25) (end 22.75 24.25) (width 0.2) (layer "B.Cu") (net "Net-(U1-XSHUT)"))
 (segment (start 24 21.35147) (end 23.024265 20.375735) (width 0.2) (layer "B.Cu") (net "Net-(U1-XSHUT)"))
 (segment (start 22.75 24.25) (end 24 23) (width 0.2) (layer "B.Cu") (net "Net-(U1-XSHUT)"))
 (segment (start 13.68 23.085) (end 14.845 24.25) (width 0.2) (layer "B.Cu") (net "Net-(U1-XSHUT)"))
 (segment (start 19.41 17) (end 15.5975 17) (width 0.2) (layer "F.Cu") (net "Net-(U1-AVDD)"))
 (segment (start 18.85 22) (end 18.1 22.75) (width 0.2) (layer "F.Cu") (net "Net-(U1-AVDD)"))
 (segment (start 19.8 22) (end 18.85 22) (width 0.2) (layer "F.Cu") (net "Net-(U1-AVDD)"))
 (segment (start 15.5975 17) (end 13.9375 18.66) (width 0.2) (layer "F.Cu") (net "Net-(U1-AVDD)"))
 (segment (start 19.41 13.825) (end 19.41 17) (width 0.2) (layer "F.Cu") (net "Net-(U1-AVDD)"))
 (via (at 13.9375 18.66) (size 0.6) (drill 0.3) (layers "F.Cu" "B.Cu") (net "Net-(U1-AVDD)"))
 (via (at 18.1 22.75) (size 0.6) (drill 0.3) (layers "F.Cu" "B.Cu") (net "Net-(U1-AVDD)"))
 (segment (start 15.33 23.085) (end 15.25 23.005) (width 0.2) (layer "B.Cu") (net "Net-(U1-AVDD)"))
 (segment (start 18.1 22.75) (end 17.765 23.085) (width 0.2) (layer "B.Cu") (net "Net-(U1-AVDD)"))
 (segment (start 15.25 19.9725) (end 13.9375 18.66) (width 0.2) (layer "B.Cu") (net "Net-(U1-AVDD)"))
 (segment (start 15.25 23.005) (end 15.25 19.9725) (width 0.2) (layer "B.Cu") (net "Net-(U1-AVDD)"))
 (segment (start 17.765 23.085) (end 15.33 23.085) (width 0.2) (layer "B.Cu") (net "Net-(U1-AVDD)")))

